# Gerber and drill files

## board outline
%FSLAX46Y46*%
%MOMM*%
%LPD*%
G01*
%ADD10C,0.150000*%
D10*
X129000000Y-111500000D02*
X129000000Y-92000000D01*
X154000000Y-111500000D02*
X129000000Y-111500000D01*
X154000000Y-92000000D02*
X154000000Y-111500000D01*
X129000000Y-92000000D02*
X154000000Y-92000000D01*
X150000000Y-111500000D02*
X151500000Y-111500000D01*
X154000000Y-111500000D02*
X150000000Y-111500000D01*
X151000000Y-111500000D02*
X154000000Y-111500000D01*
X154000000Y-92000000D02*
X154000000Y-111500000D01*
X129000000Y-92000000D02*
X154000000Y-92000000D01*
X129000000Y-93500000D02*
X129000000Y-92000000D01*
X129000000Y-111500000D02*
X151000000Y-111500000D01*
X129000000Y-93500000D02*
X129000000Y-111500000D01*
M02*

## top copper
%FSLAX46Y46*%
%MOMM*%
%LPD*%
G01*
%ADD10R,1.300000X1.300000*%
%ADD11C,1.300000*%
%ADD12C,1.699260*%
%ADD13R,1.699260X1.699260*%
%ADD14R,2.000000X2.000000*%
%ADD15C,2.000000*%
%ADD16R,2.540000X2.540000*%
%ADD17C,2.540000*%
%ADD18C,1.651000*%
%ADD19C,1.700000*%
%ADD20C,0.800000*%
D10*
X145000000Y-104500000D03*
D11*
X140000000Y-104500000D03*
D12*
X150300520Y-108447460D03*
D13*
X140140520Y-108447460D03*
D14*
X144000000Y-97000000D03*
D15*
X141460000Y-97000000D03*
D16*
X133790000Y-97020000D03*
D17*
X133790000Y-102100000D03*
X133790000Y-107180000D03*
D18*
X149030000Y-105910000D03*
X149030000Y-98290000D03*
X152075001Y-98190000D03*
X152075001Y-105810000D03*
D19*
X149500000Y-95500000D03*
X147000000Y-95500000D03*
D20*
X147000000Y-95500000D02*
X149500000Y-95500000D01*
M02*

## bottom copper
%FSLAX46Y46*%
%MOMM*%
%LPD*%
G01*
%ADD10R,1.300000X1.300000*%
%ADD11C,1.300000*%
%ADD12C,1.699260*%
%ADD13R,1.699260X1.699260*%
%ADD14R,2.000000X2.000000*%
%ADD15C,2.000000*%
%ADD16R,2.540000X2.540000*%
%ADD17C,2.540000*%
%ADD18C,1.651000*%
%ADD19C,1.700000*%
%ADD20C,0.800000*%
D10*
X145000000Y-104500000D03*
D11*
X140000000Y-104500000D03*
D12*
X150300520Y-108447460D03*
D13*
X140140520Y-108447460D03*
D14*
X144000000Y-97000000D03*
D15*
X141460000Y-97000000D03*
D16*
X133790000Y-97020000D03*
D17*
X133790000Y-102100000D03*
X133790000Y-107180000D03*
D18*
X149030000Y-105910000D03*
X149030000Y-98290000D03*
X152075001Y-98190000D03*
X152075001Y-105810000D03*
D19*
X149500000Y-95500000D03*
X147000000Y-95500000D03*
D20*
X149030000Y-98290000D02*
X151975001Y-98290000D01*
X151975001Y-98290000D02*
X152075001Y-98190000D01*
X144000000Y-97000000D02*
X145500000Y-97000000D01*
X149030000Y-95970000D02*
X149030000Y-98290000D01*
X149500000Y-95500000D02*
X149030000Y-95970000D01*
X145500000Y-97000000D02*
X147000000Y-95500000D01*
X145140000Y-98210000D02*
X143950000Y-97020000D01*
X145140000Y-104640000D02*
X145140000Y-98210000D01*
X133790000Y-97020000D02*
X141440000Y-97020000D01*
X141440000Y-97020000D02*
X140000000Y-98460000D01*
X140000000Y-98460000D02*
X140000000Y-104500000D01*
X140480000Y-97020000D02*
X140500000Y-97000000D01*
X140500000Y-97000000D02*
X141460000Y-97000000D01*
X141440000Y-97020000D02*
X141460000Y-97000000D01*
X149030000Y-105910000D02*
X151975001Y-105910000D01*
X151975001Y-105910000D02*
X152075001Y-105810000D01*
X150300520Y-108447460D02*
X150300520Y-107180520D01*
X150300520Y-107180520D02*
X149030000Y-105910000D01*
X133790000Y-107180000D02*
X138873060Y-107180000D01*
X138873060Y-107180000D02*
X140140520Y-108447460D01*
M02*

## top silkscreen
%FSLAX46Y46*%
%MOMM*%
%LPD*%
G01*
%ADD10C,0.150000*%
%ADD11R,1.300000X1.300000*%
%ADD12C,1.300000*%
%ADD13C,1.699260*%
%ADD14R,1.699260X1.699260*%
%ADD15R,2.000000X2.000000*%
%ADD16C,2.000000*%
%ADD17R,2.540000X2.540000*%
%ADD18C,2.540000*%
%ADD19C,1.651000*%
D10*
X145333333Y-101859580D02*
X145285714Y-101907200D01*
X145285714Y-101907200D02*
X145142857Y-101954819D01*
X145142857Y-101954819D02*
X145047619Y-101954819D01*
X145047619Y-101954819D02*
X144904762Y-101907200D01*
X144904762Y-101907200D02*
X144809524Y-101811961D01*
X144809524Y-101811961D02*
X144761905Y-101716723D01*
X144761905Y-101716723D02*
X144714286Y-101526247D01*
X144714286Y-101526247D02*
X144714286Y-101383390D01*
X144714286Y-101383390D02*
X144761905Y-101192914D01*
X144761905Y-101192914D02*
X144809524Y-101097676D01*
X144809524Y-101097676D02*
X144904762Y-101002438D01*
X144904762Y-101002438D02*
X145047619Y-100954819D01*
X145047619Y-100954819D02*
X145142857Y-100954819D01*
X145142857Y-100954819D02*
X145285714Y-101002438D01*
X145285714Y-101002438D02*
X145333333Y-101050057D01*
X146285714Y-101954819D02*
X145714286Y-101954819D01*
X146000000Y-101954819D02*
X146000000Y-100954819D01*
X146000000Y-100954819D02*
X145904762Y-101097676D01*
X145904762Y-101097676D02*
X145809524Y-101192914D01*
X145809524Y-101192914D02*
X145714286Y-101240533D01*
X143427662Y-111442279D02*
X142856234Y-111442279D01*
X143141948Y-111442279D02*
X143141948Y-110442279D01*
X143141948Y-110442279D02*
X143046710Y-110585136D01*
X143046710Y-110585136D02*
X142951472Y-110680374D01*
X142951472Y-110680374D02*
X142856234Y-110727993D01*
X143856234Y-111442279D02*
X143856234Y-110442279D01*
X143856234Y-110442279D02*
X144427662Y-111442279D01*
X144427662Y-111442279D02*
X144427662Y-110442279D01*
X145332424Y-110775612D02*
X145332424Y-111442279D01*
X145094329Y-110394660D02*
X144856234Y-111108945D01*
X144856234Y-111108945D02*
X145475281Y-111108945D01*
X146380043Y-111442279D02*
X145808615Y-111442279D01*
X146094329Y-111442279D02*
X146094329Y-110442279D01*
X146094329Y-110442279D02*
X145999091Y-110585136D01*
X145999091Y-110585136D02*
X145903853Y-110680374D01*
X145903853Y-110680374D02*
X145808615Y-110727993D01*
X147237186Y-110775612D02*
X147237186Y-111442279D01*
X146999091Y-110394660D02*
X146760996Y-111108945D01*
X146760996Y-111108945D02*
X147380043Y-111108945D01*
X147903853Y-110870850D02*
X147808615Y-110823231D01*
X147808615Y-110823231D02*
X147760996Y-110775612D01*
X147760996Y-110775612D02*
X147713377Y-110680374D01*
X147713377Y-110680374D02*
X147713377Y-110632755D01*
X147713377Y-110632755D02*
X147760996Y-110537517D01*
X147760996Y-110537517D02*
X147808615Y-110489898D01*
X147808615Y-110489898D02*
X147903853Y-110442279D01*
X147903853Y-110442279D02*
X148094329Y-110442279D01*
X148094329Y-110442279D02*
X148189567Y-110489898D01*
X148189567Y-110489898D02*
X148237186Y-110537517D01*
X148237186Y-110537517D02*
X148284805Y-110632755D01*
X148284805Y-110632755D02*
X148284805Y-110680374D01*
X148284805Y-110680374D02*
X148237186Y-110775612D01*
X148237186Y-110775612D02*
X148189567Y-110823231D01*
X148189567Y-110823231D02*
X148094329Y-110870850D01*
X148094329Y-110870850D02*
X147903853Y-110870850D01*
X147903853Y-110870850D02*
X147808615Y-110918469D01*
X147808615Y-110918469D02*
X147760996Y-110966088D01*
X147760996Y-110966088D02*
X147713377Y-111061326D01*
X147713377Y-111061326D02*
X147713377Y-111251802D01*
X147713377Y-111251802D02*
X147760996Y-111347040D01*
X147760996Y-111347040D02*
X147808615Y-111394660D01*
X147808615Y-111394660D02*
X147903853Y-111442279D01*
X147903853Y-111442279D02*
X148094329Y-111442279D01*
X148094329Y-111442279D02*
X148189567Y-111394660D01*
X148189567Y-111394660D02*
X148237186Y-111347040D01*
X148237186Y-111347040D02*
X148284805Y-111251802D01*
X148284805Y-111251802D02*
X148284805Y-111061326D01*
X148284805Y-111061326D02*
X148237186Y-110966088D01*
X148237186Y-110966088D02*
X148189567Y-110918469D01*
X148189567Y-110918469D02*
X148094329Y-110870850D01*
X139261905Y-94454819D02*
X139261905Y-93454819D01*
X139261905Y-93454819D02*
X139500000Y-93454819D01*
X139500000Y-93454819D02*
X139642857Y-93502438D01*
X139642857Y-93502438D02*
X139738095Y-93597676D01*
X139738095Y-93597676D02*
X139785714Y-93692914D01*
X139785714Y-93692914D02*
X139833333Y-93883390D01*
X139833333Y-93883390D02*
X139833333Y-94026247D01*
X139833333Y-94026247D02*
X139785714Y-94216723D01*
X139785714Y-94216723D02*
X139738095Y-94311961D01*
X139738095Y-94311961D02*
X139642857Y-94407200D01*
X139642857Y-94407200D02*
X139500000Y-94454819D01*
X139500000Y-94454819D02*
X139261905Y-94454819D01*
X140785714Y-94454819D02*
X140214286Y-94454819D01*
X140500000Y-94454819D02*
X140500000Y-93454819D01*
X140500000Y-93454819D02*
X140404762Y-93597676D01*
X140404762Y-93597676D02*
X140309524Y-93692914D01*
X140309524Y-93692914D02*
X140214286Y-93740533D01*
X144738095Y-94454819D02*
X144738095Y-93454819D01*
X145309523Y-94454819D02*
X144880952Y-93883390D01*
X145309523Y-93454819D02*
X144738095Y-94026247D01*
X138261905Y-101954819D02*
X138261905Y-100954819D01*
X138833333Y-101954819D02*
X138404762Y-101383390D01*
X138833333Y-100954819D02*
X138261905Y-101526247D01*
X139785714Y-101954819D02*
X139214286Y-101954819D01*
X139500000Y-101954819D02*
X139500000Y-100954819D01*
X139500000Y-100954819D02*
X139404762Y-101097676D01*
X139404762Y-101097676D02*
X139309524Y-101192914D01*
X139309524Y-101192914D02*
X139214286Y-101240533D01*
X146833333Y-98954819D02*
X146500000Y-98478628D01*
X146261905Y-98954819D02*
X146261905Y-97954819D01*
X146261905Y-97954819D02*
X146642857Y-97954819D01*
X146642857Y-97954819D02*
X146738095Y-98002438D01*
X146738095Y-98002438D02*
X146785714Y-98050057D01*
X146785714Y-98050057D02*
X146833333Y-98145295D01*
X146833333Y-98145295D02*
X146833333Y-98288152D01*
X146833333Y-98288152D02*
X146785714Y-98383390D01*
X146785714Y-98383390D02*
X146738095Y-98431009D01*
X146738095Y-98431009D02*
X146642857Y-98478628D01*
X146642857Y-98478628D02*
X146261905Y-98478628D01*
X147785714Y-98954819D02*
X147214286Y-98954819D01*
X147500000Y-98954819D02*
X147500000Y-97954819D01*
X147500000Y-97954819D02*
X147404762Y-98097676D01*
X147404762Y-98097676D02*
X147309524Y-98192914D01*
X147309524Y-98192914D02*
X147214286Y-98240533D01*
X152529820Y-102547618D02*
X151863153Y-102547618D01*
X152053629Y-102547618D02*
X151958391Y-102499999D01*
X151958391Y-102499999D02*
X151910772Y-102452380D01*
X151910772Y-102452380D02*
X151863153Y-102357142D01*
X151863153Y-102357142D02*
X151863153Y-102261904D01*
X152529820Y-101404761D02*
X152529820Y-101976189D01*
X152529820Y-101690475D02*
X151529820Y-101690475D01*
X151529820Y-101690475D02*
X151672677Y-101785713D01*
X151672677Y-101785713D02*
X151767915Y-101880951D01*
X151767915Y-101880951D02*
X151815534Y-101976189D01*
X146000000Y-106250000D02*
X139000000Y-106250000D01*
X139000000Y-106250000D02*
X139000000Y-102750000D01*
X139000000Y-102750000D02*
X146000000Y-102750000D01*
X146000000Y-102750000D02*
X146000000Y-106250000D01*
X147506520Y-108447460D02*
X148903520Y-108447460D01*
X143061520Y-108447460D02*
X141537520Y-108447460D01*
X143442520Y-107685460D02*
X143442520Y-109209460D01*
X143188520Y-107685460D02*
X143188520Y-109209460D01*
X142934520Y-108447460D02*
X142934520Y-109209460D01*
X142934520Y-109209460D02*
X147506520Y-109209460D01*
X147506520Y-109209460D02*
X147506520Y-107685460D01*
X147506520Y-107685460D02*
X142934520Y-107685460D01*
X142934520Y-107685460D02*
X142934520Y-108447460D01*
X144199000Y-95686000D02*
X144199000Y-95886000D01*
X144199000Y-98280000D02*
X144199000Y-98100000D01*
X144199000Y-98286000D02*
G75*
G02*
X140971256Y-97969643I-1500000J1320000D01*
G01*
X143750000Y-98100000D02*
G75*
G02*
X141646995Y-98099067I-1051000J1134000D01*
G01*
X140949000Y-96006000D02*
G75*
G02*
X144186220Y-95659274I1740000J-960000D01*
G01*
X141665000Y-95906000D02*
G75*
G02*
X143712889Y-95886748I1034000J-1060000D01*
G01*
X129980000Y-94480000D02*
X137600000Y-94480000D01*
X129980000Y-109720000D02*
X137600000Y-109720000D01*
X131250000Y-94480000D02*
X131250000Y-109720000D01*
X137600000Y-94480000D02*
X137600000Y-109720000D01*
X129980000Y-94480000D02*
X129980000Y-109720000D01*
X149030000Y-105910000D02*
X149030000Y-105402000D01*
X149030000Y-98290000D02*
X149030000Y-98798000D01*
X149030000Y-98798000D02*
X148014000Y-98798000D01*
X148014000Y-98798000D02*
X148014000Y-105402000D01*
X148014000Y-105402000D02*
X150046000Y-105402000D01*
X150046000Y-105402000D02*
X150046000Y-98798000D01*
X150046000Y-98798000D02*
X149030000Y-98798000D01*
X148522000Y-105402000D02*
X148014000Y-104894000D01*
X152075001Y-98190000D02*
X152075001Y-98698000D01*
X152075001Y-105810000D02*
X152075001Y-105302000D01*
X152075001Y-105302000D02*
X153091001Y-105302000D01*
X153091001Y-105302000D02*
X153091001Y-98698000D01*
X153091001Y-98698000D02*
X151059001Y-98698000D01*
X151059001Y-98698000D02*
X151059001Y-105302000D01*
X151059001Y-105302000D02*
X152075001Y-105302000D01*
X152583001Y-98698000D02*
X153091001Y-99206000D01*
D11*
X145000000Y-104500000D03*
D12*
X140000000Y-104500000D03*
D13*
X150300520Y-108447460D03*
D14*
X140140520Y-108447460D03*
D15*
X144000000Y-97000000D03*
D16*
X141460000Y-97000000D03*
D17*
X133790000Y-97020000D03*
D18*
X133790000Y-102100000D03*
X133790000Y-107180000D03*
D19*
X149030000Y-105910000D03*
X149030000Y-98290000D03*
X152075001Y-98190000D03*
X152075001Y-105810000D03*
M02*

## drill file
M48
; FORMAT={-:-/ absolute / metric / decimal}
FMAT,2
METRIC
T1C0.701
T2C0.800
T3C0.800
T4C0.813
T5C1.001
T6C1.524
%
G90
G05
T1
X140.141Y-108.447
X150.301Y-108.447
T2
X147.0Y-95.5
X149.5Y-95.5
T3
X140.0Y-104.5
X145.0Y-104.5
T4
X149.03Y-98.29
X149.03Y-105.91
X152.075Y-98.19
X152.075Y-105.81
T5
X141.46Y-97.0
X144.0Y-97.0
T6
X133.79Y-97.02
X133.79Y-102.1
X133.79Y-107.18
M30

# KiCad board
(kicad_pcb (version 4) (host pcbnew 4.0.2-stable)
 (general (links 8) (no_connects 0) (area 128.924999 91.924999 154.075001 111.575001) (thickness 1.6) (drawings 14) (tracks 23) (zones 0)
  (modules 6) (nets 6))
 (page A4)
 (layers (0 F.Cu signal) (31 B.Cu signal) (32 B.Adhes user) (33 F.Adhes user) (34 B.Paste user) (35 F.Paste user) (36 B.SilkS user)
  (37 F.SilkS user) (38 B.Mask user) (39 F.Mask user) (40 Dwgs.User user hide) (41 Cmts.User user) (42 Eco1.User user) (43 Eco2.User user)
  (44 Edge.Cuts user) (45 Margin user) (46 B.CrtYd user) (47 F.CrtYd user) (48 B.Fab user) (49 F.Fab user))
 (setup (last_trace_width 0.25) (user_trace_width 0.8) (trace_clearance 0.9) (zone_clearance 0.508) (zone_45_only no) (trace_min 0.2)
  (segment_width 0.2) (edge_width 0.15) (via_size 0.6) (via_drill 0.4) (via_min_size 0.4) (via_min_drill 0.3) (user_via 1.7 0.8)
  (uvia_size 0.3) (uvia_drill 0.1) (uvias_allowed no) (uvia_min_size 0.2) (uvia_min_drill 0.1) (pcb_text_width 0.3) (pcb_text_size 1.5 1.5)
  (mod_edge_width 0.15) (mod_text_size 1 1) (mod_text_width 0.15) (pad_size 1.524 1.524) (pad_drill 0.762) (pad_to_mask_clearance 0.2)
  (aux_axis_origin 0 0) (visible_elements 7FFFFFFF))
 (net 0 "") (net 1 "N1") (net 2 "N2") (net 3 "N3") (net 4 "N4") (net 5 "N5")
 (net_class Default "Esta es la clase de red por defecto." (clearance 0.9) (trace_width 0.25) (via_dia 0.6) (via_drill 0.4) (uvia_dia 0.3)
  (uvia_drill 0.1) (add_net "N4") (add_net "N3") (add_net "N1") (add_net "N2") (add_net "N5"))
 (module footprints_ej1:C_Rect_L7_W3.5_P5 (layer F.Cu) (at 145 104.5 180)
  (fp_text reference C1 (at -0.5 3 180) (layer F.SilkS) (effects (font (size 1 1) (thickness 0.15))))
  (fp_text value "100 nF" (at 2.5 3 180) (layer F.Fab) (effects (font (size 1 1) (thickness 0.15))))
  (fp_line (start -1 -1.75) (end 6 -1.75) (layer F.SilkS) (width 0.15))
  (fp_line (start 6 -1.75) (end 6 1.75) (layer F.SilkS) (width 0.15))
  (fp_line (start 6 1.75) (end -1 1.75) (layer F.SilkS) (width 0.15))
  (fp_line (start -1 1.75) (end -1 -1.75) (layer F.SilkS) (width 0.15))
  (pad 1 thru_hole rect (at 0 0 180) (size 1.3 1.3) (drill 0.8) (layers *.Cu *.Mask F.SilkS) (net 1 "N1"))
  (pad 2 thru_hole circle (at 5 0 180) (size 1.3 1.3) (drill 0.8) (layers *.Cu *.Mask F.SilkS) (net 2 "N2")))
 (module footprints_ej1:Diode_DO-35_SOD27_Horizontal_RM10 (layer F.Cu) (at 140.14 108.45)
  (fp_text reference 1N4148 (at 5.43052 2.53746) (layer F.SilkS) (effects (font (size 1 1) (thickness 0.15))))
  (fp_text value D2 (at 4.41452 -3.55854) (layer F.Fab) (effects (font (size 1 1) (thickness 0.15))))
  (fp_line (start 7.36652 -0.00254) (end 8.76352 -0.00254) (layer F.SilkS) (width 0.15))
  (fp_line (start 2.92152 -0.00254) (end 1.39752 -0.00254) (layer F.SilkS) (width 0.15))
  (fp_line (start 3.30252 -0.76454) (end 3.30252 0.75946) (layer F.SilkS) (width 0.15))
  (fp_line (start 3.04852 -0.76454) (end 3.04852 0.75946) (layer F.SilkS) (width 0.15))
  (fp_line (start 2.79452 -0.00254) (end 2.79452 0.75946) (layer F.SilkS) (width 0.15))
  (fp_line (start 2.79452 0.75946) (end 7.36652 0.75946) (layer F.SilkS) (width 0.15))
  (fp_line (start 7.36652 0.75946) (end 7.36652 -0.76454) (layer F.SilkS) (width 0.15))
  (fp_line (start 7.36652 -0.76454) (end 2.79452 -0.76454) (layer F.SilkS) (width 0.15))
  (fp_line (start 2.79452 -0.76454) (end 2.79452 -0.00254) (layer F.SilkS) (width 0.15))
  (pad 2 thru_hole circle (at 10.16052 -0.00254 180) (size 1.69926 1.69926) (drill 0.70104) (layers *.Cu *.Mask F.SilkS) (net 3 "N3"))
  (pad 1 thru_hole rect (at 0.00052 -0.00254 180) (size 1.69926 1.69926) (drill 0.70104) (layers *.Cu *.Mask F.SilkS) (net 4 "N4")))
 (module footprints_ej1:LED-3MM (layer F.Cu) (at 144 97 180)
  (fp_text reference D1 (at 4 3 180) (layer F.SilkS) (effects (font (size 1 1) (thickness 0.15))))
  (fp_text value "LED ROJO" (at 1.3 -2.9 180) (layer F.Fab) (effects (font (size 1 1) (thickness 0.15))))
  (fp_line (start -0.199 1.314) (end -0.199 1.114) (layer F.SilkS) (width 0.15))
  (fp_line (start -0.199 -1.28) (end -0.199 -1.1) (layer F.SilkS) (width 0.15))
  (fp_arc (start 1.301 0.034) (end -0.199 -1.286) (angle 108.5) (layer F.SilkS) (width 0.15))
  (fp_arc (start 1.301 0.034) (end 0.25 -1.1) (angle 85.7) (layer F.SilkS) (width 0.15))
  (fp_arc (start 1.311 0.034) (end 3.051 0.994) (angle 110) (layer F.SilkS) (width 0.15))
  (fp_arc (start 1.301 0.034) (end 2.335 1.094) (angle 87.5) (layer F.SilkS) (width 0.15))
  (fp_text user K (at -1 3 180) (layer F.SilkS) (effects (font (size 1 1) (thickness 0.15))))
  (pad 1 thru_hole rect (at 0 0 270) (size 2 2) (drill 1.00076) (layers *.Cu *.Mask F.SilkS) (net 1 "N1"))
  (pad 2 thru_hole circle (at 2.54 0 180) (size 2 2) (drill 1.00076) (layers *.Cu *.Mask F.SilkS) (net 2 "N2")))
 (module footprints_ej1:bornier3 (layer F.Cu) (at 133.79 102.1 270)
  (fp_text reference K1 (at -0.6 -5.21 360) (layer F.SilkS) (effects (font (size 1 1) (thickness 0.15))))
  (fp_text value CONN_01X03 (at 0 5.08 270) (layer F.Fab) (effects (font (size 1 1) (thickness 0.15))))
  (fp_line (start -7.62 3.81) (end -7.62 -3.81) (layer F.SilkS) (width 0.15))
  (fp_line (start 7.62 3.81) (end 7.62 -3.81) (layer F.SilkS) (width 0.15))
  (fp_line (start -7.62 2.54) (end 7.62 2.54) (layer F.SilkS) (width 0.15))
  (fp_line (start -7.62 -3.81) (end 7.62 -3.81) (layer F.SilkS) (width 0.15))
  (fp_line (start -7.62 3.81) (end 7.62 3.81) (layer F.SilkS) (width 0.15))
  (pad 1 thru_hole rect (at -5.08 0 270) (size 2.54 2.54) (drill 1.524) (layers *.Cu *.Mask F.SilkS) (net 2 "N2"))
  (pad 2 thru_hole circle (at 0 0 270) (size 2.54 2.54) (drill 1.524) (layers *.Cu *.Mask F.SilkS) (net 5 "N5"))
  (pad 3 thru_hole circle (at 5.08 0 270) (size 2.54 2.54) (drill 1.524) (layers *.Cu *.Mask F.SilkS) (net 4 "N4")))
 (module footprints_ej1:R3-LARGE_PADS (layer F.Cu) (at 149.03 102.1 90)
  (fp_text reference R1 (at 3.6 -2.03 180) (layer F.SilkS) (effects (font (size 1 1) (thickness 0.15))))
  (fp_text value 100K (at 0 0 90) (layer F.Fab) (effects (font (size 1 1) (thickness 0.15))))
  (fp_line (start -3.81 0) (end -3.302 0) (layer F.SilkS) (width 0.15))
  (fp_line (start 3.81 0) (end 3.302 0) (layer F.SilkS) (width 0.15))
  (fp_line (start 3.302 0) (end 3.302 -1.016) (layer F.SilkS) (width 0.15))
  (fp_line (start 3.302 -1.016) (end -3.302 -1.016) (layer F.SilkS) (width 0.15))
  (fp_line (start -3.302 -1.016) (end -3.302 1.016) (layer F.SilkS) (width 0.15))
  (fp_line (start -3.302 1.016) (end 3.302 1.016) (layer F.SilkS) (width 0.15))
  (fp_line (start 3.302 1.016) (end 3.302 0) (layer F.SilkS) (width 0.15))
  (fp_line (start -3.302 -0.508) (end -2.794 -1.016) (layer F.SilkS) (width 0.15))
  (pad 1 thru_hole circle (at -3.81 0 90) (size 1.651 1.651) (drill 0.8128) (layers *.Cu *.Mask F.SilkS) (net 3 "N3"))
  (pad 2 thru_hole circle (at 3.81 0 90) (size 1.651 1.651) (drill 0.8128) (layers *.Cu *.Mask F.SilkS) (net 1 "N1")))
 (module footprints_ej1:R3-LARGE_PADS (layer F.Cu) (at 152.075001 102 270)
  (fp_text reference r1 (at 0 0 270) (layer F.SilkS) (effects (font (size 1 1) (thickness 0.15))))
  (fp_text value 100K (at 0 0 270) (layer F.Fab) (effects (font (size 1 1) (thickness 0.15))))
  (fp_line (start -3.81 0) (end -3.302 0) (layer F.SilkS) (width 0.15))
  (fp_line (start 3.81 0) (end 3.302 0) (layer F.SilkS) (width 0.15))
  (fp_line (start 3.302 0) (end 3.302 -1.016) (layer F.SilkS) (width 0.15))
  (fp_line (start 3.302 -1.016) (end -3.302 -1.016) (layer F.SilkS) (width 0.15))
  (fp_line (start -3.302 -1.016) (end -3.302 1.016) (layer F.SilkS) (width 0.15))
  (fp_line (start -3.302 1.016) (end 3.302 1.016) (layer F.SilkS) (width 0.15))
  (fp_line (start 3.302 1.016) (end 3.302 0) (layer F.SilkS) (width 0.15))
  (fp_line (start -3.302 -0.508) (end -2.794 -1.016) (layer F.SilkS) (width 0.15))
  (pad 1 thru_hole circle (at -3.81 0 270) (size 1.651 1.651) (drill 0.8128) (layers *.Cu *.Mask F.SilkS) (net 1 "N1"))
  (pad 2 thru_hole circle (at 3.81 0 270) (size 1.651 1.651) (drill 0.8128) (layers *.Cu *.Mask F.SilkS) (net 3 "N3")))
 (gr_line (start 129 111.5) (end 129 92) (angle 90) (layer Edge.Cuts) (width 0.15))
 (gr_line (start 154 111.5) (end 129 111.5) (angle 90) (layer Edge.Cuts) (width 0.15))
 (gr_line (start 154 92) (end 154 111.5) (angle 90) (layer Edge.Cuts) (width 0.15))
 (gr_line (start 129 92) (end 154 92) (angle 90) (layer Edge.Cuts) (width 0.15))
 (gr_line (start 150 111.5) (end 151.5 111.5) (angle 90) (layer Edge.Cuts) (width 0.15))
 (gr_line (start 154 111.5) (end 150 111.5) (angle 90) (layer Edge.Cuts) (width 0.15))
 (gr_line (start 151 111.5) (end 154 111.5) (angle 90) (layer Edge.Cuts) (width 0.15))
 (gr_line (start 154 92) (end 154 111.5) (angle 90) (layer Edge.Cuts) (width 0.15))
 (gr_line (start 129 92) (end 154 92) (angle 90) (layer Edge.Cuts) (width 0.15))
 (gr_line (start 129 93.5) (end 129 92) (angle 90) (layer Edge.Cuts) (width 0.15))
 (gr_line (start 129 111.5) (end 151 111.5) (angle 90) (layer Edge.Cuts) (width 0.15))
 (gr_line (start 129 93.5) (end 129 111.5) (angle 90) (layer Edge.Cuts) (width 0.15))
 (segment (start 149.03 98.29) (end 151.975001 98.29) (width 0.8) (layer B.Cu) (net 1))
 (segment (start 151.975001 98.29) (end 152.075001 98.19) (width 0.8) (layer B.Cu) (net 1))
 (segment (start 144 97) (end 145.5 97) (width 0.8) (layer B.Cu) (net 1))
 (segment (start 149.03 95.97) (end 149.03 98.29) (width 0.8) (layer B.Cu) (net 1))
 (segment (start 149.5 95.5) (end 149.03 95.97) (width 0.8) (layer B.Cu) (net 1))
 (via (at 149.5 95.5) (size 1.7) (drill 0.8) (layers F.Cu B.Cu) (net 1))
 (segment (start 147 95.5) (end 149.5 95.5) (width 0.8) (layer F.Cu) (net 1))
 (via (at 147 95.5) (size 1.7) (drill 0.8) (layers F.Cu B.Cu) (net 1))
 (segment (start 145.5 97) (end 147 95.5) (width 0.8) (layer B.Cu) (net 1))
 (segment (start 145.14 98.21) (end 143.95 97.02) (width 0.8) (layer B.Cu) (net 1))
 (segment (start 145.14 104.64) (end 145.14 98.21) (width 0.8) (layer B.Cu) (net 1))
 (segment (start 133.79 97.02) (end 141.44 97.02) (width 0.8) (layer B.Cu) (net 2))
 (segment (start 141.44 97.02) (end 140 98.46) (width 0.8) (layer B.Cu) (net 2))
 (segment (start 140 98.46) (end 140 104.5) (width 0.8) (layer B.Cu) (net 2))
 (segment (start 140.48 97.02) (end 140.5 97) (width 0.8) (layer B.Cu) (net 2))
 (segment (start 140.5 97) (end 141.46 97) (width 0.8) (layer B.Cu) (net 2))
 (segment (start 141.44 97.02) (end 141.46 97) (width 0.8) (layer B.Cu) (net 2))
 (segment (start 149.03 105.91) (end 151.975001 105.91) (width 0.8) (layer B.Cu) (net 3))
 (segment (start 151.975001 105.91) (end 152.075001 105.81) (width 0.8) (layer B.Cu) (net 3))
 (segment (start 150.30052 108.44746) (end 150.30052 107.18052) (width 0.8) (layer B.Cu) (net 3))
 (segment (start 150.30052 107.18052) (end 149.03 105.91) (width 0.8) (layer B.Cu) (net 3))
 (segment (start 133.79 107.18) (end 138.87306 107.18) (width 0.8) (layer B.Cu) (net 4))
 (segment (start 138.87306 107.18) (end 140.14052 108.44746) (width 0.8) (layer B.Cu) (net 4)))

